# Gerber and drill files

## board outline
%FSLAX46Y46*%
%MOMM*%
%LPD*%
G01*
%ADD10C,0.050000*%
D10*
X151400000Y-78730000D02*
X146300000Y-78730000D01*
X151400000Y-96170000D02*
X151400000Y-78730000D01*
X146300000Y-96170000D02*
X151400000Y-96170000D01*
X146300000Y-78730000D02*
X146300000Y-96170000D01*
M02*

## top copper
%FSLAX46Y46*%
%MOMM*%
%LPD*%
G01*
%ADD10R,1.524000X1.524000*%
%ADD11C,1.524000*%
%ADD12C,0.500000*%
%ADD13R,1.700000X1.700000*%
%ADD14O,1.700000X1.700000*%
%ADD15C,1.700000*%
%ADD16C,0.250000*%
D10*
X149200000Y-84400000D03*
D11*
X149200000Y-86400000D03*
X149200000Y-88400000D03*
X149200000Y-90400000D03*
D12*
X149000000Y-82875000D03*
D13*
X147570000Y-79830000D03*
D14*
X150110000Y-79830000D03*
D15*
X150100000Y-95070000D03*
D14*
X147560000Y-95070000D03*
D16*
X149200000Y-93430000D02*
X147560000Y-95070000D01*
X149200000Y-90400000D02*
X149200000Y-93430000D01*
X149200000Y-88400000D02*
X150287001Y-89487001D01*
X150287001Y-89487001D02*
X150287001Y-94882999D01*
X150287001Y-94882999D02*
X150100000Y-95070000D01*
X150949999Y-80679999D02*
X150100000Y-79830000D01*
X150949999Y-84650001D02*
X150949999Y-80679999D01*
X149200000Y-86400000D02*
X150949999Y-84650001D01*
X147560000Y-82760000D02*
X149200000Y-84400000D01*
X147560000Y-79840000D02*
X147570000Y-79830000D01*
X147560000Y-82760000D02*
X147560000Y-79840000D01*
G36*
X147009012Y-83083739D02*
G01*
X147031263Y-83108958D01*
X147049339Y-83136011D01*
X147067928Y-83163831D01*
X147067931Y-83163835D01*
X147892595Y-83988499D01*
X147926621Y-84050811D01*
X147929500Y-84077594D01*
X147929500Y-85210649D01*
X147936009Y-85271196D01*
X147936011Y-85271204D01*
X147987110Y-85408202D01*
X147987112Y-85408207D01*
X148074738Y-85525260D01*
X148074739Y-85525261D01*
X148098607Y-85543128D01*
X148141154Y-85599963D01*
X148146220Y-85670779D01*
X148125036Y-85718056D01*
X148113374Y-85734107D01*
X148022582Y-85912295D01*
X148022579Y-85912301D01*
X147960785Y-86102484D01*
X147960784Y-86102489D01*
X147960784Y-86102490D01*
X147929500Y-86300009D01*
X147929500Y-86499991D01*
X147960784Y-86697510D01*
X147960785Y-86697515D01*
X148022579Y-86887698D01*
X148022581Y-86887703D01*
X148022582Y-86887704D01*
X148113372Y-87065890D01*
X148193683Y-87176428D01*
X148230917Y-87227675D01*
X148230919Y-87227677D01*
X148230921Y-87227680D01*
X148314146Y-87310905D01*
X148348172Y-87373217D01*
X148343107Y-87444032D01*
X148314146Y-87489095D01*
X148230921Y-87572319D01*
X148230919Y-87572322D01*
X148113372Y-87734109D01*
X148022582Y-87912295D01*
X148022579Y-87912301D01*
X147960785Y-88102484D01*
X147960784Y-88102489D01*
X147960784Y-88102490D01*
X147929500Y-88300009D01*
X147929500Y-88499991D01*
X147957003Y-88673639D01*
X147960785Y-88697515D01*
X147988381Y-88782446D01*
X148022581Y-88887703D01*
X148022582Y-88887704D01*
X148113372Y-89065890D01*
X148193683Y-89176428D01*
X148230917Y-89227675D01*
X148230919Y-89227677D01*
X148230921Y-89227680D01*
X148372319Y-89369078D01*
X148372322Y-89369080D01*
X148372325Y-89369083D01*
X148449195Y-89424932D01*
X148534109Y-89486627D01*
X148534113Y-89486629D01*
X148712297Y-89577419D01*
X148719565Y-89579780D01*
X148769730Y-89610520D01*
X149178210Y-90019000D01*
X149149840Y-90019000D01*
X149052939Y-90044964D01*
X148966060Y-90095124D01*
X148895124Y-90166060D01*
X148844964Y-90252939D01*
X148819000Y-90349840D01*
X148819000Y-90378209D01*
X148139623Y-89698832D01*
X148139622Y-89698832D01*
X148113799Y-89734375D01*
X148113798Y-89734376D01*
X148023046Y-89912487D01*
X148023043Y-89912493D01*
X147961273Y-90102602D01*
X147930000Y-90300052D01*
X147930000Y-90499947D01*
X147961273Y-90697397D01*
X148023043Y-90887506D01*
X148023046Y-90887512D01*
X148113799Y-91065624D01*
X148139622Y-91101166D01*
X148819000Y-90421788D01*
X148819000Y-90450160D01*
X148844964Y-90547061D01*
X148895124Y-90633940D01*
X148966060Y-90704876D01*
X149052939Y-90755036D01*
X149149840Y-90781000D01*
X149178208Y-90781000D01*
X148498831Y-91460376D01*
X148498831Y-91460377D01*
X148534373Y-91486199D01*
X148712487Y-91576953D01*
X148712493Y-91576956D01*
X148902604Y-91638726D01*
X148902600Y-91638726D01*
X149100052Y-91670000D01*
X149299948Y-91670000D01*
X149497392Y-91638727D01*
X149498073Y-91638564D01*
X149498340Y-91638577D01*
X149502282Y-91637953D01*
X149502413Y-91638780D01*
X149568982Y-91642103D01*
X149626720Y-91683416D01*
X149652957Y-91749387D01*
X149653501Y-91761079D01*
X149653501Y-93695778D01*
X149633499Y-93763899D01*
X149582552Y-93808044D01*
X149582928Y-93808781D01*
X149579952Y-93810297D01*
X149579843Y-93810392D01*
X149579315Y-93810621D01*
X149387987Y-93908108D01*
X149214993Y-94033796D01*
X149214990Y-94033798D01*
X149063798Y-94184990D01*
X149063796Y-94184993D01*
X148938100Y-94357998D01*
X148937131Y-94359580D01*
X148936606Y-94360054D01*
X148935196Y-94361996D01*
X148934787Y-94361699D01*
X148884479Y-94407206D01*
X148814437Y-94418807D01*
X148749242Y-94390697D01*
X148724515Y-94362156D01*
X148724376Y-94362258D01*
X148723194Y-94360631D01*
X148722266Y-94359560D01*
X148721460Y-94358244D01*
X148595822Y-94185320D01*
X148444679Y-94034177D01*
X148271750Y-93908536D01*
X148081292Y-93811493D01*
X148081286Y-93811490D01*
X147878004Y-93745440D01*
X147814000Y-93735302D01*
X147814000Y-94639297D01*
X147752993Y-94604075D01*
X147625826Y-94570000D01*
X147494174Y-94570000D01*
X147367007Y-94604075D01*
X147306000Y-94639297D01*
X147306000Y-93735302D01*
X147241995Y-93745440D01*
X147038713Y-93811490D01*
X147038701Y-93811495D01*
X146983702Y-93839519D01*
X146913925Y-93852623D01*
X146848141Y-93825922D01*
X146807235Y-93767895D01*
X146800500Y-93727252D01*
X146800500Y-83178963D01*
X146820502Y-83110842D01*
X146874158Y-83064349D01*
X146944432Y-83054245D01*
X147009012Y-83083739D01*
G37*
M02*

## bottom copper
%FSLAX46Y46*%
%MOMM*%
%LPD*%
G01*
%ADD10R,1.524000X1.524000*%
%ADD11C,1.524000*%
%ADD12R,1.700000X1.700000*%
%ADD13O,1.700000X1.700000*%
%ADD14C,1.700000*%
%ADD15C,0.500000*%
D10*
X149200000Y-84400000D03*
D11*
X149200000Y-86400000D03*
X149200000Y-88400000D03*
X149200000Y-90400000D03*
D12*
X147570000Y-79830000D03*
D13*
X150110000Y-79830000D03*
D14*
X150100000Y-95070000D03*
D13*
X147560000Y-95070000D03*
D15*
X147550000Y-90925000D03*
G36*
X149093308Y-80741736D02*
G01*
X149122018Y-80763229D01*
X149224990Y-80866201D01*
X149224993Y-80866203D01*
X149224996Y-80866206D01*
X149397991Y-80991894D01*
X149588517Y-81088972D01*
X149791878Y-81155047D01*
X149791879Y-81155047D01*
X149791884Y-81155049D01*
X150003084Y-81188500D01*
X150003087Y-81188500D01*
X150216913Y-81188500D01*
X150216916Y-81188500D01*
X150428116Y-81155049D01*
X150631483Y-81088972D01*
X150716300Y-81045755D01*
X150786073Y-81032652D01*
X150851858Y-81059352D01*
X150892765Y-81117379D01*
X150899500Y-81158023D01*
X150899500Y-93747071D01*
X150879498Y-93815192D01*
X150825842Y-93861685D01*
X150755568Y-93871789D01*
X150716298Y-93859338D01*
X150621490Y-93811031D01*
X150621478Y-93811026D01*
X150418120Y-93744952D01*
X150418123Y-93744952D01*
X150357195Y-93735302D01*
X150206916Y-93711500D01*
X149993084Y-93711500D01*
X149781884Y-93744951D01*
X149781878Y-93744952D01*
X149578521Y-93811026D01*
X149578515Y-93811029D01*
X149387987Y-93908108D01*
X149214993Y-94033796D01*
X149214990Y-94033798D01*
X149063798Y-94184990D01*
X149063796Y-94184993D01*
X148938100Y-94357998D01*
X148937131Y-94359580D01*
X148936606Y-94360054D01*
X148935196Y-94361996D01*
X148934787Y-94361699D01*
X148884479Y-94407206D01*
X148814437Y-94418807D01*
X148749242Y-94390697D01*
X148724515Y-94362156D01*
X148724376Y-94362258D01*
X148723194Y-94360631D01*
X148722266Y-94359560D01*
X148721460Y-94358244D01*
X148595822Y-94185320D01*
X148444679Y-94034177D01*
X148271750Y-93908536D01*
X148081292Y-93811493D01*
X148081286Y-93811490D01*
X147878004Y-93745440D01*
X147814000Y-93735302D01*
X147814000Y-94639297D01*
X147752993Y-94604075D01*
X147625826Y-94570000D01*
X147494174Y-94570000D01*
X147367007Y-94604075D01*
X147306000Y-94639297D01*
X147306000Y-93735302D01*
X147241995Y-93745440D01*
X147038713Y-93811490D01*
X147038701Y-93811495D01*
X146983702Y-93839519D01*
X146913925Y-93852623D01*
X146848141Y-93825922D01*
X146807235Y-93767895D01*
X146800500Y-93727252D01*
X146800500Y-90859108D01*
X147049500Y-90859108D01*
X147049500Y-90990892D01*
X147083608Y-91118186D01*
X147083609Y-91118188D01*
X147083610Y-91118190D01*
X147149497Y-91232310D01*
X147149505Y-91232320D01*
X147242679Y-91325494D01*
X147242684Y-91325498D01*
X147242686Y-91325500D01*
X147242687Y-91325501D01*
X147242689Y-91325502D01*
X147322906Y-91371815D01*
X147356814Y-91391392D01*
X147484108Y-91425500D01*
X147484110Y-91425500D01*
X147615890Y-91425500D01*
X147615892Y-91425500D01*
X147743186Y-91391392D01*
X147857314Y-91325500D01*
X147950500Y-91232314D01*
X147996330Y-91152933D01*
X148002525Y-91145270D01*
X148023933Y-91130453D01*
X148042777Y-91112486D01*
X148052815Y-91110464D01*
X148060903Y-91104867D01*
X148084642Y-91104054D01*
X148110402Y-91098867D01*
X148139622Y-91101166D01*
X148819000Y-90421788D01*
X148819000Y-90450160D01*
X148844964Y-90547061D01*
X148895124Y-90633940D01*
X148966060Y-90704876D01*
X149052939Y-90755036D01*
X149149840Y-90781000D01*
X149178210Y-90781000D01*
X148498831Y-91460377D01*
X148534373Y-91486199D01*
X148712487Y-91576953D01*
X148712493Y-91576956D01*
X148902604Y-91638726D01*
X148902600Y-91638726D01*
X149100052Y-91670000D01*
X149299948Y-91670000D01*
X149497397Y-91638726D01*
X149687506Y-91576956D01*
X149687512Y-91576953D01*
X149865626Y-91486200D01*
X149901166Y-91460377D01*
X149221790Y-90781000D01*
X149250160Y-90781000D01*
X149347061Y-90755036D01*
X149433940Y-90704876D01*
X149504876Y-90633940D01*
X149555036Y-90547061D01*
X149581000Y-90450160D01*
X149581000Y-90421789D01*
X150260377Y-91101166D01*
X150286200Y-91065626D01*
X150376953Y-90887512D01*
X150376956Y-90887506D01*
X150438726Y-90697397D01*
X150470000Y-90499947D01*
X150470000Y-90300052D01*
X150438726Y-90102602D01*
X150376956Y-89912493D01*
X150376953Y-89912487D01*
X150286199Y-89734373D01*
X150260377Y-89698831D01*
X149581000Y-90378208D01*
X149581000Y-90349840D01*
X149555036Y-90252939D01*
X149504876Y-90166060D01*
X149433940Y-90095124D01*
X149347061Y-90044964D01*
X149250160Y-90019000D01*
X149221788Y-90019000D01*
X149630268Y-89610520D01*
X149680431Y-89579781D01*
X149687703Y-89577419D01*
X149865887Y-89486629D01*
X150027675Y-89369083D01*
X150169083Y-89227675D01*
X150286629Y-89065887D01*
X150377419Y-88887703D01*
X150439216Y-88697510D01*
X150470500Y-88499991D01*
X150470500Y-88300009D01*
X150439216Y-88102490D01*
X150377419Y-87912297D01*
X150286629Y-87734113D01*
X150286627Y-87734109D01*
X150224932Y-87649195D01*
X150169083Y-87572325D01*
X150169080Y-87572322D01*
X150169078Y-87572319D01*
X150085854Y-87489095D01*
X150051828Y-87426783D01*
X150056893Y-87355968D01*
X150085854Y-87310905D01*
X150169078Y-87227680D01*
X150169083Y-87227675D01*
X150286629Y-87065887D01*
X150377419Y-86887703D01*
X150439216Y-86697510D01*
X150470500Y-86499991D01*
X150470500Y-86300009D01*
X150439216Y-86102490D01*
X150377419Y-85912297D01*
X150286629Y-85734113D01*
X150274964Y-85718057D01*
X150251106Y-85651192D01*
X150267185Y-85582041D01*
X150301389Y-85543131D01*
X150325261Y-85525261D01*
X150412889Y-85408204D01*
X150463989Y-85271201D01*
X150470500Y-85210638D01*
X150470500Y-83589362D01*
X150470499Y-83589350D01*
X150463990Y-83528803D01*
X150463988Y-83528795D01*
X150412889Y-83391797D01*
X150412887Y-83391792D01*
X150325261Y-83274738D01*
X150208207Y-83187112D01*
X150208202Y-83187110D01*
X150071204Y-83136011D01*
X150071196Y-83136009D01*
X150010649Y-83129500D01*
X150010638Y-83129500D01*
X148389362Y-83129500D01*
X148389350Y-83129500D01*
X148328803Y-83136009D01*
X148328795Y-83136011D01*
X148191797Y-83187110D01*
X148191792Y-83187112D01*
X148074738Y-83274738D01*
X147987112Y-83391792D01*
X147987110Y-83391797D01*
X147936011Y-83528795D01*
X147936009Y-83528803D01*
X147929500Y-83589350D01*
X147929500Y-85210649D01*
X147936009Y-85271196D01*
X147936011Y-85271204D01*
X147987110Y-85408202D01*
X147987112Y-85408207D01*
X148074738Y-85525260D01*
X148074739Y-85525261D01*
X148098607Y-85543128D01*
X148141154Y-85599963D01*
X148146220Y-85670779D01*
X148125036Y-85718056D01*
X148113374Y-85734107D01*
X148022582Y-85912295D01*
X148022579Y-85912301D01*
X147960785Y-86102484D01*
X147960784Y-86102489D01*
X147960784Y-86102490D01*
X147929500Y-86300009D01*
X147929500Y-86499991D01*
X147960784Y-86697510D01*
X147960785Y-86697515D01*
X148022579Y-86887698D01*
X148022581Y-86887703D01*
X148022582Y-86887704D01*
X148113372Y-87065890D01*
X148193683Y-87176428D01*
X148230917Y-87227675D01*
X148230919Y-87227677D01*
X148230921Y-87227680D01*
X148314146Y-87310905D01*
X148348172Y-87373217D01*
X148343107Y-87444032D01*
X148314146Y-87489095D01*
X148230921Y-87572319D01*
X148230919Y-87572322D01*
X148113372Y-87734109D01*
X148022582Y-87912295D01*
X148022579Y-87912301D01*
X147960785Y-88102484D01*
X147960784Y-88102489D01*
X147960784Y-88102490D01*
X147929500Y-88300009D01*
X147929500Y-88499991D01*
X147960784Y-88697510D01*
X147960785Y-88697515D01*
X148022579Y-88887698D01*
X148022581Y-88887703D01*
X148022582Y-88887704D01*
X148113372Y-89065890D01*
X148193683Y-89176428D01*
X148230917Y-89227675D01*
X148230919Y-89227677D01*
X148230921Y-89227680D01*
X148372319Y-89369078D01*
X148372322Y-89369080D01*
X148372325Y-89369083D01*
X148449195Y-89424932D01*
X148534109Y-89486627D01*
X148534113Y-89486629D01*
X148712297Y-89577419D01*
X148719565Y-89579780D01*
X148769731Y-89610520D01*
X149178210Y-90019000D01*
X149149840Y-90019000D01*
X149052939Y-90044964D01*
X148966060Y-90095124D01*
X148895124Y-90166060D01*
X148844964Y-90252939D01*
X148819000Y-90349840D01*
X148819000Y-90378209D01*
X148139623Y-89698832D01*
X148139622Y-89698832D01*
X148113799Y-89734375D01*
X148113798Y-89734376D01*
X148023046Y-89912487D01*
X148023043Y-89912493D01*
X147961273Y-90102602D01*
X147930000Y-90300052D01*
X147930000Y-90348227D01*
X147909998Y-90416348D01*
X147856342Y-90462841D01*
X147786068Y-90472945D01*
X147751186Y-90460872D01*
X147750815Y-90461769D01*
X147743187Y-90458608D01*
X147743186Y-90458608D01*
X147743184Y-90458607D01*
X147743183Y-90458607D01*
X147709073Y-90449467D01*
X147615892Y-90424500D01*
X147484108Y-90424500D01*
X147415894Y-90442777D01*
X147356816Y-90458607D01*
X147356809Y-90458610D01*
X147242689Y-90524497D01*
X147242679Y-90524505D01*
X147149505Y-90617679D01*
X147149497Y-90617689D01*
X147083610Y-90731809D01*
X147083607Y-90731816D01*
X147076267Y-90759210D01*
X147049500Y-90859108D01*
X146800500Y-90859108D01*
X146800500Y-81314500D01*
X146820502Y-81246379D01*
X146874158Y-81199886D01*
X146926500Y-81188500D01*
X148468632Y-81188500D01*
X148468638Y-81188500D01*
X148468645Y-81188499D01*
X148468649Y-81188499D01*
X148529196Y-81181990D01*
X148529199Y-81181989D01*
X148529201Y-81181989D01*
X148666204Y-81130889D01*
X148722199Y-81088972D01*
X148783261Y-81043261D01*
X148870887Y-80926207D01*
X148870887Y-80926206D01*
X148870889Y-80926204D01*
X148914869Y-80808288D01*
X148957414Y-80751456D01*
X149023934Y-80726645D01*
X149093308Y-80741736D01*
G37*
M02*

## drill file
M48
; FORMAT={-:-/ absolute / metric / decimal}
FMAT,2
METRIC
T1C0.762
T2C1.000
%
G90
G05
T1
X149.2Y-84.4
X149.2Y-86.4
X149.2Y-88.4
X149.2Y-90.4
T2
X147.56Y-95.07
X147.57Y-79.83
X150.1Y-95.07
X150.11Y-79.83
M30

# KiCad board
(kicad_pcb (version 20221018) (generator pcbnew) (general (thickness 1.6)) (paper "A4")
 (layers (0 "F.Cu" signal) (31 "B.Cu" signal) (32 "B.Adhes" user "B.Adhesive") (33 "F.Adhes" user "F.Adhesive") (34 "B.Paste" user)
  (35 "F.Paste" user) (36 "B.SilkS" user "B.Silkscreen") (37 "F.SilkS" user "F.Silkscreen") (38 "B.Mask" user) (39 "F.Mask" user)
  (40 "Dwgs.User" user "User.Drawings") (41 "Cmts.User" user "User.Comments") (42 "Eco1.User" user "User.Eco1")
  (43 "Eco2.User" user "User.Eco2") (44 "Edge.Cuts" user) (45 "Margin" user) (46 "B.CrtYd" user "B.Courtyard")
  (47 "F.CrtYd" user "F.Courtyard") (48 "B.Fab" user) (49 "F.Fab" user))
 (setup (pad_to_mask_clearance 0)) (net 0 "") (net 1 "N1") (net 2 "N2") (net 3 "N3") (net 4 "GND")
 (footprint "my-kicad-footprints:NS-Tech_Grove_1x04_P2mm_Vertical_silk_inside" (layer "F.Cu") (at 149.2 84.4)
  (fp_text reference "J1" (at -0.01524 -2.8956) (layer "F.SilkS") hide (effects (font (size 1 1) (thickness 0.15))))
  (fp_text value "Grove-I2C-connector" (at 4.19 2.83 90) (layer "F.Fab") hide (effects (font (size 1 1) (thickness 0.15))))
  (pad "1" thru_hole rect (at 0 0) (size 1.524 1.524) (drill 0.762) (layers "*.Cu" "*.Mask") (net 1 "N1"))
  (pad "2" thru_hole circle (at 0 2) (size 1.524 1.524) (drill 0.762) (layers "*.Cu" "*.Mask") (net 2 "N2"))
  (pad "3" thru_hole circle (at 0 4) (size 1.524 1.524) (drill 0.762) (layers "*.Cu" "*.Mask") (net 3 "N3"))
  (pad "4" thru_hole circle (at 0 6) (size 1.524 1.524) (drill 0.762) (layers "*.Cu" "*.Mask") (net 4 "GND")))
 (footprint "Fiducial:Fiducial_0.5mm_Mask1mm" (layer "F.Cu") (at 149 82.875)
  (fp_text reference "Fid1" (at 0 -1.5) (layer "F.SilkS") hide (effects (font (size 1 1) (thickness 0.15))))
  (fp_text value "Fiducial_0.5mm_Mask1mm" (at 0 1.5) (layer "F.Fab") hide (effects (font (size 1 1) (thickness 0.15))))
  (pad "" smd circle (at 0 0) (size 0.5 0.5) (layers "F.Cu" "F.Mask") (solder_mask_margin 0.25) (clearance 0.25)))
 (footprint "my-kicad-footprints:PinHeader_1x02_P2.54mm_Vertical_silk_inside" (layer "B.Cu") (at 147.57 79.83 -90)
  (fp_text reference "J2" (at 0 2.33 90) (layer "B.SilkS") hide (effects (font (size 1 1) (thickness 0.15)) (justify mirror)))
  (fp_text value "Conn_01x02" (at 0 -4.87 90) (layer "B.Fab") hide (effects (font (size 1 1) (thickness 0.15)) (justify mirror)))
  (pad "1" thru_hole rect (at 0 0 270) (size 1.7 1.7) (drill 1) (layers "*.Cu" "*.Mask") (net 1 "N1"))
  (pad "2" thru_hole oval (at 0 -2.54 270) (size 1.7 1.7) (drill 1) (layers "*.Cu" "*.Mask") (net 2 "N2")))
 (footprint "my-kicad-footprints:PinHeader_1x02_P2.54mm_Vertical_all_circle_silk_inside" (layer "B.Cu") (at 150.1 95.07 90)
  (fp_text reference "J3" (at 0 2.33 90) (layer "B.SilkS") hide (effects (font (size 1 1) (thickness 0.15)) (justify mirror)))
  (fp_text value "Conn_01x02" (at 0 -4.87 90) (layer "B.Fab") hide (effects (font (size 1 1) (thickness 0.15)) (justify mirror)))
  (pad "1" thru_hole circle (at 0 0 90) (size 1.7 1.7) (drill 1) (layers "*.Cu" "*.Mask") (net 3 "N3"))
  (pad "2" thru_hole oval (at 0 -2.54 90) (size 1.7 1.7) (drill 1) (layers "*.Cu" "*.Mask") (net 4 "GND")))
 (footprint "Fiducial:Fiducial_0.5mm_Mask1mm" (layer "B.Cu") (at 147.55 90.925)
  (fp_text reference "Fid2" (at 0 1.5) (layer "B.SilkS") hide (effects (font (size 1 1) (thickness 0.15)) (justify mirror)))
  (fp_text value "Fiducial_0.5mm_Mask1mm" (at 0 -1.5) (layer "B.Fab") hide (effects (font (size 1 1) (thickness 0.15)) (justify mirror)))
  (pad "" smd circle (at 0 0) (size 0.5 0.5) (layers "B.Cu" "B.Mask") (solder_mask_margin 0.25) (clearance 0.25)))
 (gr_line (start 151.4 78.73) (end 146.3 78.73) (stroke (width 0.05) (type solid)) (layer "Edge.Cuts"))
 (gr_line (start 151.4 96.17) (end 151.4 78.73) (stroke (width 0.05) (type solid)) (layer "Edge.Cuts"))
 (gr_line (start 146.3 96.17) (end 151.4 96.17) (stroke (width 0.05) (type solid)) (layer "Edge.Cuts"))
 (gr_line (start 146.3 78.73) (end 146.3 96.17) (stroke (width 0.05) (type solid)) (layer "Edge.Cuts"))
 (segment (start 149.2 93.43) (end 147.56 95.07) (width 0.25) (layer "F.Cu") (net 4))
 (segment (start 149.2 90.4) (end 149.2 93.43) (width 0.25) (layer "F.Cu") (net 4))
 (segment (start 149.2 88.4) (end 150.287001 89.487001) (width 0.25) (layer "F.Cu") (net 3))
 (segment (start 150.287001 89.487001) (end 150.287001 94.882999) (width 0.25) (layer "F.Cu") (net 3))
 (segment (start 150.287001 94.882999) (end 150.1 95.07) (width 0.25) (layer "F.Cu") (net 3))
 (segment (start 150.949999 80.679999) (end 150.1 79.83) (width 0.25) (layer "F.Cu") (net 2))
 (segment (start 150.949999 84.650001) (end 150.949999 80.679999) (width 0.25) (layer "F.Cu") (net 2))
 (segment (start 149.2 86.4) (end 150.949999 84.650001) (width 0.25) (layer "F.Cu") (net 2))
 (segment (start 147.56 82.76) (end 149.2 84.4) (width 0.25) (layer "F.Cu") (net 1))
 (segment (start 147.56 79.84) (end 147.57 79.83) (width 0.25) (layer "F.Cu") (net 1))
 (segment (start 147.56 82.76) (end 147.56 79.84) (width 0.25) (layer "F.Cu") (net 1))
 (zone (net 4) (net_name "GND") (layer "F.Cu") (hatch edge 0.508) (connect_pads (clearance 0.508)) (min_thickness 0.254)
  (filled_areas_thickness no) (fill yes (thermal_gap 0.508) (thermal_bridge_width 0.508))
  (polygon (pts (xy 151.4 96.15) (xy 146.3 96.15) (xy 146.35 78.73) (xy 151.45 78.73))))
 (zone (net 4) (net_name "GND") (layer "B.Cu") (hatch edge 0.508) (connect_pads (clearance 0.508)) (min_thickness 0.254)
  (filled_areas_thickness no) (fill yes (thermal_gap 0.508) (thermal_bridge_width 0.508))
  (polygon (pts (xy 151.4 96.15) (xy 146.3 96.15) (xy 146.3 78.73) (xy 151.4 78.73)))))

